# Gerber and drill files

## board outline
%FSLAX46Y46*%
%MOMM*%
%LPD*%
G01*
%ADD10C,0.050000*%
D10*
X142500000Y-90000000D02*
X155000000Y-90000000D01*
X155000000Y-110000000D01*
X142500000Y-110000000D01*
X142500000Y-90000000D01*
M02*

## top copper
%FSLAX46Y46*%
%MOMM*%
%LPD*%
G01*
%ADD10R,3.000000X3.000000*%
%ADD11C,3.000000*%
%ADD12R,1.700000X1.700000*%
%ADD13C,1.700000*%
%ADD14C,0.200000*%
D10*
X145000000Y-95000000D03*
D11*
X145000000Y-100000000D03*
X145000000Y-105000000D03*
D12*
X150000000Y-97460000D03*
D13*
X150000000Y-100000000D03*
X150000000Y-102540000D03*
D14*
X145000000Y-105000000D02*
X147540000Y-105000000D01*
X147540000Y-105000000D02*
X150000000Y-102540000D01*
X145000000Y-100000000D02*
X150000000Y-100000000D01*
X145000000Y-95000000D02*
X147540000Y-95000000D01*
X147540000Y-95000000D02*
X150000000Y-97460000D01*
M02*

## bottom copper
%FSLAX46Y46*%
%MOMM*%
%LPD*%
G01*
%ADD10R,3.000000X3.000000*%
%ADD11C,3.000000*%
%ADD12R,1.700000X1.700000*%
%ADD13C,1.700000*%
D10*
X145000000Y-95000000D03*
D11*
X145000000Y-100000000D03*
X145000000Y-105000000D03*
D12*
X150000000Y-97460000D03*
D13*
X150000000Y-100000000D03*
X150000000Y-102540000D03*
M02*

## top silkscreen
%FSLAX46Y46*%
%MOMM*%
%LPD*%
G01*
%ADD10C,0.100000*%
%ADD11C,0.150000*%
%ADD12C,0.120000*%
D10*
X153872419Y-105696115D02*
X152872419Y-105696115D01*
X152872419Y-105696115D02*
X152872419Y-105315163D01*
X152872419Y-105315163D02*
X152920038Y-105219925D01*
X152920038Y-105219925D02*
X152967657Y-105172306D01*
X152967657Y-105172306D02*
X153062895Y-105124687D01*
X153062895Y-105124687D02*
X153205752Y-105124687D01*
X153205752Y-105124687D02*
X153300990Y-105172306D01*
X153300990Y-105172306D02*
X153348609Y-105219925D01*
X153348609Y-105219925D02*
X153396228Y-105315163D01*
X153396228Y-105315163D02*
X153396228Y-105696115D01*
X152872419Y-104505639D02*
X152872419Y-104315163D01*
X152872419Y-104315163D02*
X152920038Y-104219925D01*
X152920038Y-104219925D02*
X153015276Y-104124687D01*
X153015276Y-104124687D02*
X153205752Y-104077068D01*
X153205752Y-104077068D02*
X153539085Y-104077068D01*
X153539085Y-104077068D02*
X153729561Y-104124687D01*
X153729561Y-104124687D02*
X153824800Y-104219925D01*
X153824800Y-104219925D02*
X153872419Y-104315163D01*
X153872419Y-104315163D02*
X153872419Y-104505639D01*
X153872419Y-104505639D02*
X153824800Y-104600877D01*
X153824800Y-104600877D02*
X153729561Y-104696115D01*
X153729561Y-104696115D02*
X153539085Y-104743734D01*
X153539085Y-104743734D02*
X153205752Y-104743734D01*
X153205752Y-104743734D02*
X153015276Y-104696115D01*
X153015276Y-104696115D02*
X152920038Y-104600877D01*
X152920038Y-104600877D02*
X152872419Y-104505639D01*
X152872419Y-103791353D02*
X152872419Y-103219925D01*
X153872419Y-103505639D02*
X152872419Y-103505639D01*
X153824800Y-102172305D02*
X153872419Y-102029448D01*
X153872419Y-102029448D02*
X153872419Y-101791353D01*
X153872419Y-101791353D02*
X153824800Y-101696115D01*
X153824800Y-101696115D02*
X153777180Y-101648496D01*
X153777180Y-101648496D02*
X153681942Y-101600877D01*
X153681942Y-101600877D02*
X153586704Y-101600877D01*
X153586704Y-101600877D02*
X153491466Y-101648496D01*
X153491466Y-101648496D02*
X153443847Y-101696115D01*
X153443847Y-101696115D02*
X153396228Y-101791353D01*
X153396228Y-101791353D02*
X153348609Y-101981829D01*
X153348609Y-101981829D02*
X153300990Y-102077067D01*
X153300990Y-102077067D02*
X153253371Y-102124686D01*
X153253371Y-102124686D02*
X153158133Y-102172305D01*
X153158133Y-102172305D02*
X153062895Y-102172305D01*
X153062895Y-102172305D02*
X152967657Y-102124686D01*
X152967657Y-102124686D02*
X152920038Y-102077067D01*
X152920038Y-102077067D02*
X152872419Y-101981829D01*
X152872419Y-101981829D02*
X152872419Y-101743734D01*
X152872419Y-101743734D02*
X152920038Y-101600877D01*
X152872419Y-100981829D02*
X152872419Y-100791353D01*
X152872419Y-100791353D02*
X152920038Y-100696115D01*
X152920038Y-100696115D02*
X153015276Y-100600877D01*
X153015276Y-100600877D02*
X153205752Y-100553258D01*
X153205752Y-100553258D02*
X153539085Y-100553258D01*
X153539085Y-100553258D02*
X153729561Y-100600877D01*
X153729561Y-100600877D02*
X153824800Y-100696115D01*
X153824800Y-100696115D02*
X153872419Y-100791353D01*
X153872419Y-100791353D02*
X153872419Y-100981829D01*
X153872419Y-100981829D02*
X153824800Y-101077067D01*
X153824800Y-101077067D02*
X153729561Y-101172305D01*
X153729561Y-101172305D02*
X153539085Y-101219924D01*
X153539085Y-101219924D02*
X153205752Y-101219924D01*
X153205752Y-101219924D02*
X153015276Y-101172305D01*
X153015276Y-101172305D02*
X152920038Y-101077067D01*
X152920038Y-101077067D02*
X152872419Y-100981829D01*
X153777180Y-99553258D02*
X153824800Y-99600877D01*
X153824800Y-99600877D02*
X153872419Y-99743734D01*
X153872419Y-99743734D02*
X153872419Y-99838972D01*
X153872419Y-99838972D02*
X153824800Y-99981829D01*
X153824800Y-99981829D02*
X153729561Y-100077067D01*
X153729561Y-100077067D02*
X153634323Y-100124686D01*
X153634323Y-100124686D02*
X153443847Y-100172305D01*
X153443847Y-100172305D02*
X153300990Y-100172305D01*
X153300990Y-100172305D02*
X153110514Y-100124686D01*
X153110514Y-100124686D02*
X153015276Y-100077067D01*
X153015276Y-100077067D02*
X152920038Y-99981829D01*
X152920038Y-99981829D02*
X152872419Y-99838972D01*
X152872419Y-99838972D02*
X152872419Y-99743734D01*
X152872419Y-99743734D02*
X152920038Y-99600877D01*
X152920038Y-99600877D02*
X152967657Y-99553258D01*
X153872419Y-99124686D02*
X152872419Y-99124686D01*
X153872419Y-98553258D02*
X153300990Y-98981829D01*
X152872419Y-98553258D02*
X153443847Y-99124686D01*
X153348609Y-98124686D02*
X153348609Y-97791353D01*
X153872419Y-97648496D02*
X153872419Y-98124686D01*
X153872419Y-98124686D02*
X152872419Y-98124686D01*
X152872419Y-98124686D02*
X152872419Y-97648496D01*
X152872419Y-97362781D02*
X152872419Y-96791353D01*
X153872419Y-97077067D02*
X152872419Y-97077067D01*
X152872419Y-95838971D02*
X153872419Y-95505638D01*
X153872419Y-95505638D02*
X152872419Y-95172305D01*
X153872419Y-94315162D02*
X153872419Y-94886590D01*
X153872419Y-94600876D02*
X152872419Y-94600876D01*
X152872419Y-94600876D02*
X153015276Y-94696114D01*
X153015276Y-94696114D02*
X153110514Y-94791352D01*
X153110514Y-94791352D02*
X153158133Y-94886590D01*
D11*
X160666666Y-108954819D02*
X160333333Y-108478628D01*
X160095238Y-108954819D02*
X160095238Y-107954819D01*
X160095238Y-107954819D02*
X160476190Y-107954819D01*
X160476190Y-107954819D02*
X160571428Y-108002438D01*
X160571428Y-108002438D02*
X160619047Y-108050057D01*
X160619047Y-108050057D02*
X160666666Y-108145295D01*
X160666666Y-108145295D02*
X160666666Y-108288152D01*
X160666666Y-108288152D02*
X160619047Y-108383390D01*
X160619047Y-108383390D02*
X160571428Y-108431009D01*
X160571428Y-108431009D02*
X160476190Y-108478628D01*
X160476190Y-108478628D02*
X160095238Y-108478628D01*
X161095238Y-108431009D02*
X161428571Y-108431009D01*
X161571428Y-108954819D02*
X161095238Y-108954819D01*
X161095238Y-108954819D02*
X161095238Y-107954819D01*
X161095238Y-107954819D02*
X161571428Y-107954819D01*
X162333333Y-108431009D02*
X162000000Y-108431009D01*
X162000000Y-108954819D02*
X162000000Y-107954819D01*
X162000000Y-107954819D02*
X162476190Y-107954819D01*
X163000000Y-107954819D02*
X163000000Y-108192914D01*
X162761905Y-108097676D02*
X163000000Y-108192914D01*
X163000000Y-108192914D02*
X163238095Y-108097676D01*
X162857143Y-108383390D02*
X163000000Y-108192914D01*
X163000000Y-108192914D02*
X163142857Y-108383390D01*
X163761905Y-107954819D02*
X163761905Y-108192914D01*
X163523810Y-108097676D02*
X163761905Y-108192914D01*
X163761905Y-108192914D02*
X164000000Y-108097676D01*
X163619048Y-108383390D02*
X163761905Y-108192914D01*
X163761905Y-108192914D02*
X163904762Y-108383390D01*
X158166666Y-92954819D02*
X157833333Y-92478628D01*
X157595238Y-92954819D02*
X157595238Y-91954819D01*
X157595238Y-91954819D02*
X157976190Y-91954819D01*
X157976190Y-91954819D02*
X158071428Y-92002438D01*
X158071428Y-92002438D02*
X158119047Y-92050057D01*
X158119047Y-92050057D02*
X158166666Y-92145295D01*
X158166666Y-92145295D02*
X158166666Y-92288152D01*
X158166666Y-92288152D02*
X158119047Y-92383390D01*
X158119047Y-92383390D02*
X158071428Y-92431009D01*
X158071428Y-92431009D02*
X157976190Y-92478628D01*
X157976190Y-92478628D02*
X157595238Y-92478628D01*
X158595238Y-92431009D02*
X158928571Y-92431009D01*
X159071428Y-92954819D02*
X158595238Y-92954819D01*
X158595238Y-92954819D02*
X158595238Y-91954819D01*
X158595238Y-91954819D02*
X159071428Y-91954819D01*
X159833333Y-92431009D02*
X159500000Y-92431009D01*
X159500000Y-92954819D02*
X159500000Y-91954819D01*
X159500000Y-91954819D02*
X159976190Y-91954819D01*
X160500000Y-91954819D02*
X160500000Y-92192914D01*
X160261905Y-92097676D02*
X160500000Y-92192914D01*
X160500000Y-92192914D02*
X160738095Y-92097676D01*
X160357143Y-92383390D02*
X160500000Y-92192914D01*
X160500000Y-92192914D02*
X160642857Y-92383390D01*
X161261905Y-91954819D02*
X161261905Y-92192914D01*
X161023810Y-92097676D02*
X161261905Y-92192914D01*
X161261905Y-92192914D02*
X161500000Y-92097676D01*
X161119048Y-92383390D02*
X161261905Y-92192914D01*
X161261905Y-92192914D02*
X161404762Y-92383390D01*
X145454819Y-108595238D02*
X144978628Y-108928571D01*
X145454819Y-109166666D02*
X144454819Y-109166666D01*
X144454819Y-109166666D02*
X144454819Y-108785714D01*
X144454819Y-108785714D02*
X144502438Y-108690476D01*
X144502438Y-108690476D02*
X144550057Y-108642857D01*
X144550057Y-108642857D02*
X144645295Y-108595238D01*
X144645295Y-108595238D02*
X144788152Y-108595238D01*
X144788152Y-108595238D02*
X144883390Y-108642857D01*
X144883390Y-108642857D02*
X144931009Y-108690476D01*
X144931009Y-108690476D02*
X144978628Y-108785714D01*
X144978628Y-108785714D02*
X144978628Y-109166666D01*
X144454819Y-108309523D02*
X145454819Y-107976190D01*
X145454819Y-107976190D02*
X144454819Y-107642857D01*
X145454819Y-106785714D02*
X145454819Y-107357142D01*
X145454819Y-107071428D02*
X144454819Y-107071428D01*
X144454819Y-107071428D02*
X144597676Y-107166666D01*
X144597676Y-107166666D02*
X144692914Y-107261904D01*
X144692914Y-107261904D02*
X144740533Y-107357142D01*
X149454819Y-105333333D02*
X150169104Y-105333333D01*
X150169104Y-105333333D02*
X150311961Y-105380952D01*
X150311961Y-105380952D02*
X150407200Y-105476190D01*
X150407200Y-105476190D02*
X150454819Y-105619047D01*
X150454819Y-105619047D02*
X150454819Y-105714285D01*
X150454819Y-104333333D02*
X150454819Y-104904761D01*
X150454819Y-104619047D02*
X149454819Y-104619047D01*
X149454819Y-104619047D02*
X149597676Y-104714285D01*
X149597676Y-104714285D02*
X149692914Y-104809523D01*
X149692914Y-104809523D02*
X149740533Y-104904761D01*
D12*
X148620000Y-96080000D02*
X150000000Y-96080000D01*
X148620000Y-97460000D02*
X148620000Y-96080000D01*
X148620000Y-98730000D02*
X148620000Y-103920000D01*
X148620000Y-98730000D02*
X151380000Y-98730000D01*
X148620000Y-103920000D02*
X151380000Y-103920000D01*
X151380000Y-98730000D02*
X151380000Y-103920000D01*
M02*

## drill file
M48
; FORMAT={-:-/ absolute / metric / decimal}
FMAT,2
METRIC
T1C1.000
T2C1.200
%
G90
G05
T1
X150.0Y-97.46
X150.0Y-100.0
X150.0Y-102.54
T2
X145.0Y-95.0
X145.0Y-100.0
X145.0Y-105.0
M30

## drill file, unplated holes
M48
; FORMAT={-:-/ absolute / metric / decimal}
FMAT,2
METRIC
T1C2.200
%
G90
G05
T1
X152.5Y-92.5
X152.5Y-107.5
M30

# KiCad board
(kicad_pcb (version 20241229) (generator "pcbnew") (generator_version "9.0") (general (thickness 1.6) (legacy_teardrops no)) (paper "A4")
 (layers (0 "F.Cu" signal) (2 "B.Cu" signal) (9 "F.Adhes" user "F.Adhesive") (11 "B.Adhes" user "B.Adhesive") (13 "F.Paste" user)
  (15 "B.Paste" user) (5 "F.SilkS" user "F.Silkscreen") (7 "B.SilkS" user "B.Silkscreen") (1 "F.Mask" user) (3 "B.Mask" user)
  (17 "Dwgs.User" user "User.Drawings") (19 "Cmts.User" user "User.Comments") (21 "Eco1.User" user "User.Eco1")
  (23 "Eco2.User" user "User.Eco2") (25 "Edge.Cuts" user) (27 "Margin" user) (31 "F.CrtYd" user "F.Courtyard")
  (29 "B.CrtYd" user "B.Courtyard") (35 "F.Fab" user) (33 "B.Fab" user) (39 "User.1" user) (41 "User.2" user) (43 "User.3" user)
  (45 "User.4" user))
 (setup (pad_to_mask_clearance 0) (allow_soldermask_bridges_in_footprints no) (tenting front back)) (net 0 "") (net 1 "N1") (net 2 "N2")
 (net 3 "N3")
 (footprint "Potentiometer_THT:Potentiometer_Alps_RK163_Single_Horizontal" (layer "F.Cu") (at 145 95)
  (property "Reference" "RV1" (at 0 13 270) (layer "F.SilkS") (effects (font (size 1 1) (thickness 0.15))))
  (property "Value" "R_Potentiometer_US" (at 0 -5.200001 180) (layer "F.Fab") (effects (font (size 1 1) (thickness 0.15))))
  (pad "1" thru_hole rect (at 0 0 180) (size 3 3) (drill 1.2) (layers "*.Cu" "*.Mask") (remove_unused_layers no) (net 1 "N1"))
  (pad "2" thru_hole circle (at 0 5 180) (size 3 3) (drill 1.2) (layers "*.Cu" "*.Mask") (remove_unused_layers no) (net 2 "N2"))
  (pad "3" thru_hole circle (at 0 10 180) (size 3 3) (drill 1.2) (layers "*.Cu" "*.Mask") (remove_unused_layers no) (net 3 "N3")))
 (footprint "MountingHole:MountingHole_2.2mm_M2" (layer "F.Cu") (at 152.5 92.5)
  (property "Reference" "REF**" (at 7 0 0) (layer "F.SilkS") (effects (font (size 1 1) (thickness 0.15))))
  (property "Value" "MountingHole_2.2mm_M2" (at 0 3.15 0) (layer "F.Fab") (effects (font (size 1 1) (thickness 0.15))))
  (pad "" np_thru_hole circle (at 0 0) (size 2.2 2.2) (drill 2.2) (layers "*.Cu" "*.Mask")))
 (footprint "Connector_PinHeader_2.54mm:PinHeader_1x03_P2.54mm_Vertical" (layer "F.Cu") (at 150 97.46)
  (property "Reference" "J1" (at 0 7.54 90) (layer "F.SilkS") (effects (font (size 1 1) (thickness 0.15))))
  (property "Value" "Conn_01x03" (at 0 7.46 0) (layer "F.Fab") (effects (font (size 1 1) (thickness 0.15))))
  (fp_line (start -1.38 -1.38) (end 0 -1.38) (stroke (width 0.12) (type solid)) (layer "F.SilkS"))
  (fp_line (start -1.38 0) (end -1.38 -1.38) (stroke (width 0.12) (type solid)) (layer "F.SilkS"))
  (fp_line (start -1.38 1.27) (end -1.38 6.46) (stroke (width 0.12) (type solid)) (layer "F.SilkS"))
  (fp_line (start -1.38 1.27) (end 1.38 1.27) (stroke (width 0.12) (type solid)) (layer "F.SilkS"))
  (fp_line (start -1.38 6.46) (end 1.38 6.46) (stroke (width 0.12) (type solid)) (layer "F.SilkS"))
  (fp_line (start 1.38 1.27) (end 1.38 6.46) (stroke (width 0.12) (type solid)) (layer "F.SilkS"))
  (pad "1" thru_hole rect (at 0 0) (size 1.7 1.7) (drill 1) (layers "*.Cu" "*.Mask") (remove_unused_layers no) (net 1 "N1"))
  (pad "2" thru_hole circle (at 0 2.54) (size 1.7 1.7) (drill 1) (layers "*.Cu" "*.Mask") (remove_unused_layers no) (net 2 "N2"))
  (pad "3" thru_hole circle (at 0 5.08) (size 1.7 1.7) (drill 1) (layers "*.Cu" "*.Mask") (remove_unused_layers no) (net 3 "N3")))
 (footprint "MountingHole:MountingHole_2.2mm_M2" (layer "F.Cu") (at 152.5 107.5)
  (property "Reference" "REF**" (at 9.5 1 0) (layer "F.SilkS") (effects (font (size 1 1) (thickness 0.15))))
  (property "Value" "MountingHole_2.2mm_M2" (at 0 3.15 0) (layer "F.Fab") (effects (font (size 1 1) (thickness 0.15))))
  (pad "" np_thru_hole circle (at 0 0) (size 2.2 2.2) (drill 2.2) (layers "*.Cu" "*.Mask")))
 (gr_rect (start 142.5 90) (end 155 110) (stroke (width 0.05) (type default)) (fill no) (layer "Edge.Cuts"))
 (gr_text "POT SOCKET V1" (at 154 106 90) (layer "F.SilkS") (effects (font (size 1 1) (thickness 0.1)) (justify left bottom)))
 (segment (start 147.54 105) (end 150 102.54) (width 0.2) (layer "F.Cu") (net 3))
 (segment (start 145 105) (end 147.54 105) (width 0.2) (layer "F.Cu") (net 3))
 (segment (start 145 100) (end 150 100) (width 0.2) (layer "F.Cu") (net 2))
 (segment (start 147.54 95) (end 150 97.46) (width 0.2) (layer "F.Cu") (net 1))
 (segment (start 145 95) (end 147.54 95) (width 0.2) (layer "F.Cu") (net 1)))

